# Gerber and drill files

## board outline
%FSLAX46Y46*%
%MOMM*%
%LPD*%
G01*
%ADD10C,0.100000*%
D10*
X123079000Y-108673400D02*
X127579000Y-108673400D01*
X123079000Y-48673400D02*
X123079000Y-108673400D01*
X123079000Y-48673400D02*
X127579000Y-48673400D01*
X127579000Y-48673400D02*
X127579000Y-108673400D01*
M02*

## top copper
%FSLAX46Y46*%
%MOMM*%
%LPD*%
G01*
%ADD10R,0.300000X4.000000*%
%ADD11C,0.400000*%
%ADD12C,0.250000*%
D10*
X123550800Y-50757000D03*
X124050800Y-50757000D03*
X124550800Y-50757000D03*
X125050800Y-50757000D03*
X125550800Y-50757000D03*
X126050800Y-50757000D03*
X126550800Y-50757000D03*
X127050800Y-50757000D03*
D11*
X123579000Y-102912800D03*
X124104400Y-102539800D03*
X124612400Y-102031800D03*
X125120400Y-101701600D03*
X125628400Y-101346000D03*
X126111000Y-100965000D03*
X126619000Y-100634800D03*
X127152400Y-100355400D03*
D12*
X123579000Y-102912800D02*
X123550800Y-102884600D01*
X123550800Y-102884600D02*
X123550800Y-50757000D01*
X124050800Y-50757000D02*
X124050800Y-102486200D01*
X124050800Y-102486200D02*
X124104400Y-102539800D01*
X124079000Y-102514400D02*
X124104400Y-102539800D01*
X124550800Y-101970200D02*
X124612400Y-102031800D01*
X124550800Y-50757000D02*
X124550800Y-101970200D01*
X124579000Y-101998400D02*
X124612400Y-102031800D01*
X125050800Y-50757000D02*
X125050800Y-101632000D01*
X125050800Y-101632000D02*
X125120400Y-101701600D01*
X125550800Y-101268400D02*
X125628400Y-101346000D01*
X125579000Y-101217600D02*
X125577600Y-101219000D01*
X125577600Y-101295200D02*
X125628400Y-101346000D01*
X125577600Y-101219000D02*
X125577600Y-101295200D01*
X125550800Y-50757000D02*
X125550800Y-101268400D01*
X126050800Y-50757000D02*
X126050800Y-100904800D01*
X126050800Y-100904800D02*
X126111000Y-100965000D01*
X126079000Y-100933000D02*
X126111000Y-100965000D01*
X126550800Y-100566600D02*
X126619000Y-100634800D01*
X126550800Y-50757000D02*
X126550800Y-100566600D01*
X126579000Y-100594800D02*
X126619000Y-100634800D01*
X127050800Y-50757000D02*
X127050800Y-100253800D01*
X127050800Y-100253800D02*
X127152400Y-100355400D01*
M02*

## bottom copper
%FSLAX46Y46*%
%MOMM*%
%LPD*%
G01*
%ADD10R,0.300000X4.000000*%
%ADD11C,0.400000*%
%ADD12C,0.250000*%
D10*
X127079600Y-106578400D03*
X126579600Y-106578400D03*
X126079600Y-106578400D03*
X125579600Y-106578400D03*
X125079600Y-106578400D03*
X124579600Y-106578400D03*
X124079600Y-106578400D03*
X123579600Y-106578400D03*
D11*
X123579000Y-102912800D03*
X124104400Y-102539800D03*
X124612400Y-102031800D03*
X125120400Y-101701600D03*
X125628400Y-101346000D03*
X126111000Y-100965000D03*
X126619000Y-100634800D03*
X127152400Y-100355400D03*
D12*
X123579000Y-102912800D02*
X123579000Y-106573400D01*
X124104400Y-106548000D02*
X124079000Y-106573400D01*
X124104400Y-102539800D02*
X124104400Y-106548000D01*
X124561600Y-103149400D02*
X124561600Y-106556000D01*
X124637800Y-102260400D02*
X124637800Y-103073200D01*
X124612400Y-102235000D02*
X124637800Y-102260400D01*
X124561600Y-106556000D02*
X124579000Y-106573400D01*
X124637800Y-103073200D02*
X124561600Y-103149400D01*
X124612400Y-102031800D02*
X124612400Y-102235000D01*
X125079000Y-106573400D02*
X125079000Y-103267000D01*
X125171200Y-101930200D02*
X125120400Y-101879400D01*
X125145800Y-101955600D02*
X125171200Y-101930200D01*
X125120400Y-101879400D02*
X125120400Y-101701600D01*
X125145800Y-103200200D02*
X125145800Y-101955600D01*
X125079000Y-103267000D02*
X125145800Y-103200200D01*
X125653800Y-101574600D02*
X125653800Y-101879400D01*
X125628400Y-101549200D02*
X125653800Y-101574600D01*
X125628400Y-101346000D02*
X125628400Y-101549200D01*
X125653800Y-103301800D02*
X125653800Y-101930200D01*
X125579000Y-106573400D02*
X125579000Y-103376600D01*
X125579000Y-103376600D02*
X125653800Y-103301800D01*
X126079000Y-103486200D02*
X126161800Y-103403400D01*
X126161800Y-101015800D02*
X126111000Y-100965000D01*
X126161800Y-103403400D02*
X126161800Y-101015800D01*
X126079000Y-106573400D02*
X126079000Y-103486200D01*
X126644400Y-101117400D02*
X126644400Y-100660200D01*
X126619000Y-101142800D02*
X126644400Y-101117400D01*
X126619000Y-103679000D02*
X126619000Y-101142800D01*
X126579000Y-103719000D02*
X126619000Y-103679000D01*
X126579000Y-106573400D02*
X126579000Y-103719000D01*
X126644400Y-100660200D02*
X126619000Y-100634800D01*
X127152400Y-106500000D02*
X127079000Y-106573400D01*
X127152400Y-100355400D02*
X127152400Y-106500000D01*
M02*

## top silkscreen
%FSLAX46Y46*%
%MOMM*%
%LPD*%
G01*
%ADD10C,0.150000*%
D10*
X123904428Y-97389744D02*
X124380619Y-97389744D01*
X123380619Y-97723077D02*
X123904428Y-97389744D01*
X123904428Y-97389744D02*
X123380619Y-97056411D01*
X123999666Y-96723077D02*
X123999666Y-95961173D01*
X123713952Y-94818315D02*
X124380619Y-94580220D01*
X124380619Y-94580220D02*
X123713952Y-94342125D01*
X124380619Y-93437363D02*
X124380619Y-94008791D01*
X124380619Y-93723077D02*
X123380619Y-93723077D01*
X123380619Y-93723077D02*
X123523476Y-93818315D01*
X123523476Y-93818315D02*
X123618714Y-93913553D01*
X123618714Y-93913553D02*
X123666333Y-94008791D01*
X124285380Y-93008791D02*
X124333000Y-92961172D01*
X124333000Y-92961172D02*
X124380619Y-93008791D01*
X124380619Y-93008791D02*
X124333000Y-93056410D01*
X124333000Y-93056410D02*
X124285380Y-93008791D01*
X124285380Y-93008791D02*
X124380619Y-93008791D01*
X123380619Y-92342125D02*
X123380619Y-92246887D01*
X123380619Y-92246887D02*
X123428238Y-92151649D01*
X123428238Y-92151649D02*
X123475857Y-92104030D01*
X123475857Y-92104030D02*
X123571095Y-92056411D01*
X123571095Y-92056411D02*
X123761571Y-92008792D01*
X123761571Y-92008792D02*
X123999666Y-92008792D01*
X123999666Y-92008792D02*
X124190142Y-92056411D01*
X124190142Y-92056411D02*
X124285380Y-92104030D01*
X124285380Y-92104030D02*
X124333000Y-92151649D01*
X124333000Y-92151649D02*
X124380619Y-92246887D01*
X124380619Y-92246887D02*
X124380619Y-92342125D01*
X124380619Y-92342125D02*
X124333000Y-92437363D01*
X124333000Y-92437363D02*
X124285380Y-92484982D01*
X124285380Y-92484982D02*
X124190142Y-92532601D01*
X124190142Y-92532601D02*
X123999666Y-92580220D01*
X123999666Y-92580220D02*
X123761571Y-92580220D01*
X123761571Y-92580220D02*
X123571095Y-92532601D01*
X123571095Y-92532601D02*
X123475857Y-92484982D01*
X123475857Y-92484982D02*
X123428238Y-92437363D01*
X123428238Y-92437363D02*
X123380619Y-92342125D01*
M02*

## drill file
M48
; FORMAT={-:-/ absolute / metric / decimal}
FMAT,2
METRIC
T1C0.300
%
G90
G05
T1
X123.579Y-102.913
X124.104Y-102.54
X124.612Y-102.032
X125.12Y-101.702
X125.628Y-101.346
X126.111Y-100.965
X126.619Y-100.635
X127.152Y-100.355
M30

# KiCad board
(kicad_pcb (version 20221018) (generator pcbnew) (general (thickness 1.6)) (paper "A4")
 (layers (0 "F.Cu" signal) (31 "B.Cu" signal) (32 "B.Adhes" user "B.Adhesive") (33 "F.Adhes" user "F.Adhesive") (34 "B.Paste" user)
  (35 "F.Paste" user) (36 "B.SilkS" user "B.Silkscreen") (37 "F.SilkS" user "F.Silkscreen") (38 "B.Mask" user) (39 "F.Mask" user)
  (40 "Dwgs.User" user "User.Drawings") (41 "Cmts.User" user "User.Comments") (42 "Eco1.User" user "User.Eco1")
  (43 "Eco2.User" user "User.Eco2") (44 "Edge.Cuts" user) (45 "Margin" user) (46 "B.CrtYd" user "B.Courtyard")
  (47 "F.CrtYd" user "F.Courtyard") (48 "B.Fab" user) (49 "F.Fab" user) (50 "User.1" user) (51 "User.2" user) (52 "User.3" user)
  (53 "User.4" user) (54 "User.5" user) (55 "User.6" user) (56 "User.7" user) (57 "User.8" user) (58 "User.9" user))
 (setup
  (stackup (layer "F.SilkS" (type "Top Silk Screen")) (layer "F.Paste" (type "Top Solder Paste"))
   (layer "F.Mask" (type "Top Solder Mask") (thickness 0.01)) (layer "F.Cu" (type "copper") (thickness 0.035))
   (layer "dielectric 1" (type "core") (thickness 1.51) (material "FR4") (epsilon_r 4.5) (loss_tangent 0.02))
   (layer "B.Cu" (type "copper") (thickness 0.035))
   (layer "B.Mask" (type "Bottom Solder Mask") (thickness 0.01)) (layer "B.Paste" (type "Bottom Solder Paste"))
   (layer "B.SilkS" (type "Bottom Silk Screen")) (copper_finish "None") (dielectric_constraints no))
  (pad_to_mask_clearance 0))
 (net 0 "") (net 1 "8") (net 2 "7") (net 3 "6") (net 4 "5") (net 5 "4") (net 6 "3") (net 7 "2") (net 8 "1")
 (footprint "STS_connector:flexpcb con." (layer "F.Cu") (at 123.0508 52.757)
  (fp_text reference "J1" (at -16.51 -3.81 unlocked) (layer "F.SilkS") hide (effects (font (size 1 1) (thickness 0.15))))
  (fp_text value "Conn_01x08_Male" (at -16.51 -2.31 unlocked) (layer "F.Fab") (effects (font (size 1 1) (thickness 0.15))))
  (pad "1" smd rect (at 0.5 -2) (size 0.3 4) (layers "F.Cu" "F.Paste" "F.Mask") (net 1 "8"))
  (pad "2" smd rect (at 1 -2) (size 0.3 4) (layers "F.Cu" "F.Paste" "F.Mask") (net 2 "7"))
  (pad "3" smd rect (at 1.5 -2) (size 0.3 4) (layers "F.Cu" "F.Paste" "F.Mask") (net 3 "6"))
  (pad "4" smd rect (at 2 -2) (size 0.3 4) (layers "F.Cu" "F.Paste" "F.Mask") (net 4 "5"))
  (pad "5" smd rect (at 2.5 -2) (size 0.3 4) (layers "F.Cu" "F.Paste" "F.Mask") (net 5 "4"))
  (pad "6" smd rect (at 3 -2) (size 0.3 4) (layers "F.Cu" "F.Paste" "F.Mask") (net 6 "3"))
  (pad "7" smd rect (at 3.5 -2) (size 0.3 4) (layers "F.Cu" "F.Paste" "F.Mask") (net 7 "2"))
  (pad "8" smd rect (at 4 -2) (size 0.3 4) (layers "F.Cu" "F.Paste" "F.Mask") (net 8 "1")))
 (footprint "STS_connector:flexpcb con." (layer "B.Cu") (at 127.5796 108.5784 180)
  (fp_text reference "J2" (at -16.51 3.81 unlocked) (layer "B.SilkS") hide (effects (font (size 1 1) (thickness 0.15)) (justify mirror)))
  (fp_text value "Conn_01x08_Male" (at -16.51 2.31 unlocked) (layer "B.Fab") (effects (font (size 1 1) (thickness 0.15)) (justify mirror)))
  (pad "1" smd rect (at 0.5 2 180) (size 0.3 4) (layers "B.Cu" "B.Paste" "B.Mask") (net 8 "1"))
  (pad "2" smd rect (at 1 2 180) (size 0.3 4) (layers "B.Cu" "B.Paste" "B.Mask") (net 7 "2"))
  (pad "3" smd rect (at 1.5 2 180) (size 0.3 4) (layers "B.Cu" "B.Paste" "B.Mask") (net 6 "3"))
  (pad "4" smd rect (at 2 2 180) (size 0.3 4) (layers "B.Cu" "B.Paste" "B.Mask") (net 5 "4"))
  (pad "5" smd rect (at 2.5 2 180) (size 0.3 4) (layers "B.Cu" "B.Paste" "B.Mask") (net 4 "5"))
  (pad "6" smd rect (at 3 2 180) (size 0.3 4) (layers "B.Cu" "B.Paste" "B.Mask") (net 3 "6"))
  (pad "7" smd rect (at 3.5 2 180) (size 0.3 4) (layers "B.Cu" "B.Paste" "B.Mask") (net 2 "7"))
  (pad "8" smd rect (at 4 2 180) (size 0.3 4) (layers "B.Cu" "B.Paste" "B.Mask") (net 1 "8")))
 (gr_line (start 123.079 108.6734) (end 127.579 108.6734) (stroke (width 0.1) (type solid)) (layer "Edge.Cuts"))
 (gr_line (start 123.079 48.6734) (end 123.079 108.6734) (stroke (width 0.1) (type solid)) (layer "Edge.Cuts"))
 (gr_line (start 123.079 48.6734) (end 127.579 48.6734) (stroke (width 0.1) (type solid)) (layer "Edge.Cuts"))
 (gr_line (start 127.579 48.6734) (end 127.579 108.6734) (stroke (width 0.1) (type solid)) (layer "Edge.Cuts"))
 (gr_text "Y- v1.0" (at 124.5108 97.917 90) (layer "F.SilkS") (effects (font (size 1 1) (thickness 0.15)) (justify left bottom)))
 (segment (start 123.579 102.9128) (end 123.5508 102.8846) (width 0.25) (layer "F.Cu") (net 1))
 (segment (start 123.5508 102.8846) (end 123.5508 50.757) (width 0.25) (layer "F.Cu") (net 1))
 (via (at 123.579 102.9128) (size 0.4) (drill 0.3) (layers "F.Cu" "B.Cu") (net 1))
 (segment (start 123.579 102.9128) (end 123.579 106.5734) (width 0.25) (layer "B.Cu") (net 1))
 (segment (start 124.0508 50.757) (end 124.0508 102.4862) (width 0.25) (layer "F.Cu") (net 2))
 (segment (start 124.0508 102.4862) (end 124.1044 102.5398) (width 0.25) (layer "F.Cu") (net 2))
 (segment (start 124.079 102.5144) (end 124.1044 102.5398) (width 0.25) (layer "F.Cu") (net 2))
 (via (at 124.1044 102.5398) (size 0.4) (drill 0.3) (layers "F.Cu" "B.Cu") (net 2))
 (segment (start 124.1044 106.548) (end 124.079 106.5734) (width 0.25) (layer "B.Cu") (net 2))
 (segment (start 124.1044 102.5398) (end 124.1044 106.548) (width 0.25) (layer "B.Cu") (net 2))
 (segment (start 124.5508 101.9702) (end 124.6124 102.0318) (width 0.25) (layer "F.Cu") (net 3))
 (segment (start 124.5508 50.757) (end 124.5508 101.9702) (width 0.25) (layer "F.Cu") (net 3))
 (segment (start 124.579 101.9984) (end 124.6124 102.0318) (width 0.25) (layer "F.Cu") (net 3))
 (via (at 124.6124 102.0318) (size 0.4) (drill 0.3) (layers "F.Cu" "B.Cu") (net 3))
 (segment (start 124.5616 103.1494) (end 124.5616 106.556) (width 0.25) (layer "B.Cu") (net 3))
 (segment (start 124.6378 102.2604) (end 124.6378 103.0732) (width 0.25) (layer "B.Cu") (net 3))
 (segment (start 124.6124 102.235) (end 124.6378 102.2604) (width 0.25) (layer "B.Cu") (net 3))
 (segment (start 124.5616 106.556) (end 124.579 106.5734) (width 0.25) (layer "B.Cu") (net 3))
 (segment (start 124.6378 103.0732) (end 124.5616 103.1494) (width 0.25) (layer "B.Cu") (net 3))
 (segment (start 124.6124 102.0318) (end 124.6124 102.235) (width 0.25) (layer "B.Cu") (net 3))
 (segment (start 125.0508 50.757) (end 125.0508 101.632) (width 0.25) (layer "F.Cu") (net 4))
 (segment (start 125.0508 101.632) (end 125.1204 101.7016) (width 0.25) (layer "F.Cu") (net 4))
 (via (at 125.1204 101.7016) (size 0.4) (drill 0.3) (layers "F.Cu" "B.Cu") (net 4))
 (segment (start 125.079 106.5734) (end 125.079 103.267) (width 0.25) (layer "B.Cu") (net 4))
 (segment (start 125.1712 101.9302) (end 125.1204 101.8794) (width 0.25) (layer "B.Cu") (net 4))
 (segment (start 125.1458 101.9556) (end 125.1712 101.9302) (width 0.25) (layer "B.Cu") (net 4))
 (segment (start 125.1204 101.8794) (end 125.1204 101.7016) (width 0.25) (layer "B.Cu") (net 4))
 (segment (start 125.1458 103.2002) (end 125.1458 101.9556) (width 0.25) (layer "B.Cu") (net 4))
 (segment (start 125.079 103.267) (end 125.1458 103.2002) (width 0.25) (layer "B.Cu") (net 4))
 (segment (start 125.5508 101.2684) (end 125.6284 101.346) (width 0.25) (layer "F.Cu") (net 5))
 (segment (start 125.579 101.2176) (end 125.5776 101.219) (width 0.25) (layer "F.Cu") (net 5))
 (segment (start 125.5776 101.2952) (end 125.6284 101.346) (width 0.25) (layer "F.Cu") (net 5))
 (segment (start 125.5776 101.219) (end 125.5776 101.2952) (width 0.25) (layer "F.Cu") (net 5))
 (segment (start 125.5508 50.757) (end 125.5508 101.2684) (width 0.25) (layer "F.Cu") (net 5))
 (via (at 125.6284 101.346) (size 0.4) (drill 0.3) (layers "F.Cu" "B.Cu") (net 5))
 (segment (start 125.6538 101.5746) (end 125.6538 101.8794) (width 0.25) (layer "B.Cu") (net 5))
 (segment (start 125.6284 101.5492) (end 125.6538 101.5746) (width 0.25) (layer "B.Cu") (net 5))
 (segment (start 125.6284 101.346) (end 125.6284 101.5492) (width 0.25) (layer "B.Cu") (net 5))
 (segment (start 125.6538 103.3018) (end 125.6538 101.9302) (width 0.25) (layer "B.Cu") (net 5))
 (segment (start 125.579 106.5734) (end 125.579 103.3766) (width 0.25) (layer "B.Cu") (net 5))
 (segment (start 125.579 103.3766) (end 125.6538 103.3018) (width 0.25) (layer "B.Cu") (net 5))
 (segment (start 126.0508 50.757) (end 126.0508 100.9048) (width 0.25) (layer "F.Cu") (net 6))
 (segment (start 126.0508 100.9048) (end 126.111 100.965) (width 0.25) (layer "F.Cu") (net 6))
 (segment (start 126.079 100.933) (end 126.111 100.965) (width 0.25) (layer "F.Cu") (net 6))
 (via (at 126.111 100.965) (size 0.4) (drill 0.3) (layers "F.Cu" "B.Cu") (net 6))
 (segment (start 126.079 103.4862) (end 126.1618 103.4034) (width 0.25) (layer "B.Cu") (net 6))
 (segment (start 126.1618 101.0158) (end 126.111 100.965) (width 0.25) (layer "B.Cu") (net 6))
 (segment (start 126.1618 103.4034) (end 126.1618 101.0158) (width 0.25) (layer "B.Cu") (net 6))
 (segment (start 126.079 106.5734) (end 126.079 103.4862) (width 0.25) (layer "B.Cu") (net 6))
 (segment (start 126.5508 100.5666) (end 126.619 100.6348) (width 0.25) (layer "F.Cu") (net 7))
 (segment (start 126.5508 50.757) (end 126.5508 100.5666) (width 0.25) (layer "F.Cu") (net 7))
 (segment (start 126.579 100.5948) (end 126.619 100.6348) (width 0.25) (layer "F.Cu") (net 7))
 (via (at 126.619 100.6348) (size 0.4) (drill 0.3) (layers "F.Cu" "B.Cu") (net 7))
 (segment (start 126.6444 101.1174) (end 126.6444 100.6602) (width 0.25) (layer "B.Cu") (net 7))
 (segment (start 126.619 101.1428) (end 126.6444 101.1174) (width 0.25) (layer "B.Cu") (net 7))
 (segment (start 126.619 103.679) (end 126.619 101.1428) (width 0.25) (layer "B.Cu") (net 7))
 (segment (start 126.579 103.719) (end 126.619 103.679) (width 0.25) (layer "B.Cu") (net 7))
 (segment (start 126.579 106.5734) (end 126.579 103.719) (width 0.25) (layer "B.Cu") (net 7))
 (segment (start 126.6444 100.6602) (end 126.619 100.6348) (width 0.25) (layer "B.Cu") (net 7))
 (segment (start 127.0508 50.757) (end 127.0508 100.2538) (width 0.25) (layer "F.Cu") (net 8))
 (segment (start 127.0508 100.2538) (end 127.1524 100.3554) (width 0.25) (layer "F.Cu") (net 8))
 (via (at 127.1524 100.3554) (size 0.4) (drill 0.3) (layers "F.Cu" "B.Cu") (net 8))
 (segment (start 127.1524 106.5) (end 127.079 106.5734) (width 0.25) (layer "B.Cu") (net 8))
 (segment (start 127.1524 100.3554) (end 127.1524 106.5) (width 0.25) (layer "B.Cu") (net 8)))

